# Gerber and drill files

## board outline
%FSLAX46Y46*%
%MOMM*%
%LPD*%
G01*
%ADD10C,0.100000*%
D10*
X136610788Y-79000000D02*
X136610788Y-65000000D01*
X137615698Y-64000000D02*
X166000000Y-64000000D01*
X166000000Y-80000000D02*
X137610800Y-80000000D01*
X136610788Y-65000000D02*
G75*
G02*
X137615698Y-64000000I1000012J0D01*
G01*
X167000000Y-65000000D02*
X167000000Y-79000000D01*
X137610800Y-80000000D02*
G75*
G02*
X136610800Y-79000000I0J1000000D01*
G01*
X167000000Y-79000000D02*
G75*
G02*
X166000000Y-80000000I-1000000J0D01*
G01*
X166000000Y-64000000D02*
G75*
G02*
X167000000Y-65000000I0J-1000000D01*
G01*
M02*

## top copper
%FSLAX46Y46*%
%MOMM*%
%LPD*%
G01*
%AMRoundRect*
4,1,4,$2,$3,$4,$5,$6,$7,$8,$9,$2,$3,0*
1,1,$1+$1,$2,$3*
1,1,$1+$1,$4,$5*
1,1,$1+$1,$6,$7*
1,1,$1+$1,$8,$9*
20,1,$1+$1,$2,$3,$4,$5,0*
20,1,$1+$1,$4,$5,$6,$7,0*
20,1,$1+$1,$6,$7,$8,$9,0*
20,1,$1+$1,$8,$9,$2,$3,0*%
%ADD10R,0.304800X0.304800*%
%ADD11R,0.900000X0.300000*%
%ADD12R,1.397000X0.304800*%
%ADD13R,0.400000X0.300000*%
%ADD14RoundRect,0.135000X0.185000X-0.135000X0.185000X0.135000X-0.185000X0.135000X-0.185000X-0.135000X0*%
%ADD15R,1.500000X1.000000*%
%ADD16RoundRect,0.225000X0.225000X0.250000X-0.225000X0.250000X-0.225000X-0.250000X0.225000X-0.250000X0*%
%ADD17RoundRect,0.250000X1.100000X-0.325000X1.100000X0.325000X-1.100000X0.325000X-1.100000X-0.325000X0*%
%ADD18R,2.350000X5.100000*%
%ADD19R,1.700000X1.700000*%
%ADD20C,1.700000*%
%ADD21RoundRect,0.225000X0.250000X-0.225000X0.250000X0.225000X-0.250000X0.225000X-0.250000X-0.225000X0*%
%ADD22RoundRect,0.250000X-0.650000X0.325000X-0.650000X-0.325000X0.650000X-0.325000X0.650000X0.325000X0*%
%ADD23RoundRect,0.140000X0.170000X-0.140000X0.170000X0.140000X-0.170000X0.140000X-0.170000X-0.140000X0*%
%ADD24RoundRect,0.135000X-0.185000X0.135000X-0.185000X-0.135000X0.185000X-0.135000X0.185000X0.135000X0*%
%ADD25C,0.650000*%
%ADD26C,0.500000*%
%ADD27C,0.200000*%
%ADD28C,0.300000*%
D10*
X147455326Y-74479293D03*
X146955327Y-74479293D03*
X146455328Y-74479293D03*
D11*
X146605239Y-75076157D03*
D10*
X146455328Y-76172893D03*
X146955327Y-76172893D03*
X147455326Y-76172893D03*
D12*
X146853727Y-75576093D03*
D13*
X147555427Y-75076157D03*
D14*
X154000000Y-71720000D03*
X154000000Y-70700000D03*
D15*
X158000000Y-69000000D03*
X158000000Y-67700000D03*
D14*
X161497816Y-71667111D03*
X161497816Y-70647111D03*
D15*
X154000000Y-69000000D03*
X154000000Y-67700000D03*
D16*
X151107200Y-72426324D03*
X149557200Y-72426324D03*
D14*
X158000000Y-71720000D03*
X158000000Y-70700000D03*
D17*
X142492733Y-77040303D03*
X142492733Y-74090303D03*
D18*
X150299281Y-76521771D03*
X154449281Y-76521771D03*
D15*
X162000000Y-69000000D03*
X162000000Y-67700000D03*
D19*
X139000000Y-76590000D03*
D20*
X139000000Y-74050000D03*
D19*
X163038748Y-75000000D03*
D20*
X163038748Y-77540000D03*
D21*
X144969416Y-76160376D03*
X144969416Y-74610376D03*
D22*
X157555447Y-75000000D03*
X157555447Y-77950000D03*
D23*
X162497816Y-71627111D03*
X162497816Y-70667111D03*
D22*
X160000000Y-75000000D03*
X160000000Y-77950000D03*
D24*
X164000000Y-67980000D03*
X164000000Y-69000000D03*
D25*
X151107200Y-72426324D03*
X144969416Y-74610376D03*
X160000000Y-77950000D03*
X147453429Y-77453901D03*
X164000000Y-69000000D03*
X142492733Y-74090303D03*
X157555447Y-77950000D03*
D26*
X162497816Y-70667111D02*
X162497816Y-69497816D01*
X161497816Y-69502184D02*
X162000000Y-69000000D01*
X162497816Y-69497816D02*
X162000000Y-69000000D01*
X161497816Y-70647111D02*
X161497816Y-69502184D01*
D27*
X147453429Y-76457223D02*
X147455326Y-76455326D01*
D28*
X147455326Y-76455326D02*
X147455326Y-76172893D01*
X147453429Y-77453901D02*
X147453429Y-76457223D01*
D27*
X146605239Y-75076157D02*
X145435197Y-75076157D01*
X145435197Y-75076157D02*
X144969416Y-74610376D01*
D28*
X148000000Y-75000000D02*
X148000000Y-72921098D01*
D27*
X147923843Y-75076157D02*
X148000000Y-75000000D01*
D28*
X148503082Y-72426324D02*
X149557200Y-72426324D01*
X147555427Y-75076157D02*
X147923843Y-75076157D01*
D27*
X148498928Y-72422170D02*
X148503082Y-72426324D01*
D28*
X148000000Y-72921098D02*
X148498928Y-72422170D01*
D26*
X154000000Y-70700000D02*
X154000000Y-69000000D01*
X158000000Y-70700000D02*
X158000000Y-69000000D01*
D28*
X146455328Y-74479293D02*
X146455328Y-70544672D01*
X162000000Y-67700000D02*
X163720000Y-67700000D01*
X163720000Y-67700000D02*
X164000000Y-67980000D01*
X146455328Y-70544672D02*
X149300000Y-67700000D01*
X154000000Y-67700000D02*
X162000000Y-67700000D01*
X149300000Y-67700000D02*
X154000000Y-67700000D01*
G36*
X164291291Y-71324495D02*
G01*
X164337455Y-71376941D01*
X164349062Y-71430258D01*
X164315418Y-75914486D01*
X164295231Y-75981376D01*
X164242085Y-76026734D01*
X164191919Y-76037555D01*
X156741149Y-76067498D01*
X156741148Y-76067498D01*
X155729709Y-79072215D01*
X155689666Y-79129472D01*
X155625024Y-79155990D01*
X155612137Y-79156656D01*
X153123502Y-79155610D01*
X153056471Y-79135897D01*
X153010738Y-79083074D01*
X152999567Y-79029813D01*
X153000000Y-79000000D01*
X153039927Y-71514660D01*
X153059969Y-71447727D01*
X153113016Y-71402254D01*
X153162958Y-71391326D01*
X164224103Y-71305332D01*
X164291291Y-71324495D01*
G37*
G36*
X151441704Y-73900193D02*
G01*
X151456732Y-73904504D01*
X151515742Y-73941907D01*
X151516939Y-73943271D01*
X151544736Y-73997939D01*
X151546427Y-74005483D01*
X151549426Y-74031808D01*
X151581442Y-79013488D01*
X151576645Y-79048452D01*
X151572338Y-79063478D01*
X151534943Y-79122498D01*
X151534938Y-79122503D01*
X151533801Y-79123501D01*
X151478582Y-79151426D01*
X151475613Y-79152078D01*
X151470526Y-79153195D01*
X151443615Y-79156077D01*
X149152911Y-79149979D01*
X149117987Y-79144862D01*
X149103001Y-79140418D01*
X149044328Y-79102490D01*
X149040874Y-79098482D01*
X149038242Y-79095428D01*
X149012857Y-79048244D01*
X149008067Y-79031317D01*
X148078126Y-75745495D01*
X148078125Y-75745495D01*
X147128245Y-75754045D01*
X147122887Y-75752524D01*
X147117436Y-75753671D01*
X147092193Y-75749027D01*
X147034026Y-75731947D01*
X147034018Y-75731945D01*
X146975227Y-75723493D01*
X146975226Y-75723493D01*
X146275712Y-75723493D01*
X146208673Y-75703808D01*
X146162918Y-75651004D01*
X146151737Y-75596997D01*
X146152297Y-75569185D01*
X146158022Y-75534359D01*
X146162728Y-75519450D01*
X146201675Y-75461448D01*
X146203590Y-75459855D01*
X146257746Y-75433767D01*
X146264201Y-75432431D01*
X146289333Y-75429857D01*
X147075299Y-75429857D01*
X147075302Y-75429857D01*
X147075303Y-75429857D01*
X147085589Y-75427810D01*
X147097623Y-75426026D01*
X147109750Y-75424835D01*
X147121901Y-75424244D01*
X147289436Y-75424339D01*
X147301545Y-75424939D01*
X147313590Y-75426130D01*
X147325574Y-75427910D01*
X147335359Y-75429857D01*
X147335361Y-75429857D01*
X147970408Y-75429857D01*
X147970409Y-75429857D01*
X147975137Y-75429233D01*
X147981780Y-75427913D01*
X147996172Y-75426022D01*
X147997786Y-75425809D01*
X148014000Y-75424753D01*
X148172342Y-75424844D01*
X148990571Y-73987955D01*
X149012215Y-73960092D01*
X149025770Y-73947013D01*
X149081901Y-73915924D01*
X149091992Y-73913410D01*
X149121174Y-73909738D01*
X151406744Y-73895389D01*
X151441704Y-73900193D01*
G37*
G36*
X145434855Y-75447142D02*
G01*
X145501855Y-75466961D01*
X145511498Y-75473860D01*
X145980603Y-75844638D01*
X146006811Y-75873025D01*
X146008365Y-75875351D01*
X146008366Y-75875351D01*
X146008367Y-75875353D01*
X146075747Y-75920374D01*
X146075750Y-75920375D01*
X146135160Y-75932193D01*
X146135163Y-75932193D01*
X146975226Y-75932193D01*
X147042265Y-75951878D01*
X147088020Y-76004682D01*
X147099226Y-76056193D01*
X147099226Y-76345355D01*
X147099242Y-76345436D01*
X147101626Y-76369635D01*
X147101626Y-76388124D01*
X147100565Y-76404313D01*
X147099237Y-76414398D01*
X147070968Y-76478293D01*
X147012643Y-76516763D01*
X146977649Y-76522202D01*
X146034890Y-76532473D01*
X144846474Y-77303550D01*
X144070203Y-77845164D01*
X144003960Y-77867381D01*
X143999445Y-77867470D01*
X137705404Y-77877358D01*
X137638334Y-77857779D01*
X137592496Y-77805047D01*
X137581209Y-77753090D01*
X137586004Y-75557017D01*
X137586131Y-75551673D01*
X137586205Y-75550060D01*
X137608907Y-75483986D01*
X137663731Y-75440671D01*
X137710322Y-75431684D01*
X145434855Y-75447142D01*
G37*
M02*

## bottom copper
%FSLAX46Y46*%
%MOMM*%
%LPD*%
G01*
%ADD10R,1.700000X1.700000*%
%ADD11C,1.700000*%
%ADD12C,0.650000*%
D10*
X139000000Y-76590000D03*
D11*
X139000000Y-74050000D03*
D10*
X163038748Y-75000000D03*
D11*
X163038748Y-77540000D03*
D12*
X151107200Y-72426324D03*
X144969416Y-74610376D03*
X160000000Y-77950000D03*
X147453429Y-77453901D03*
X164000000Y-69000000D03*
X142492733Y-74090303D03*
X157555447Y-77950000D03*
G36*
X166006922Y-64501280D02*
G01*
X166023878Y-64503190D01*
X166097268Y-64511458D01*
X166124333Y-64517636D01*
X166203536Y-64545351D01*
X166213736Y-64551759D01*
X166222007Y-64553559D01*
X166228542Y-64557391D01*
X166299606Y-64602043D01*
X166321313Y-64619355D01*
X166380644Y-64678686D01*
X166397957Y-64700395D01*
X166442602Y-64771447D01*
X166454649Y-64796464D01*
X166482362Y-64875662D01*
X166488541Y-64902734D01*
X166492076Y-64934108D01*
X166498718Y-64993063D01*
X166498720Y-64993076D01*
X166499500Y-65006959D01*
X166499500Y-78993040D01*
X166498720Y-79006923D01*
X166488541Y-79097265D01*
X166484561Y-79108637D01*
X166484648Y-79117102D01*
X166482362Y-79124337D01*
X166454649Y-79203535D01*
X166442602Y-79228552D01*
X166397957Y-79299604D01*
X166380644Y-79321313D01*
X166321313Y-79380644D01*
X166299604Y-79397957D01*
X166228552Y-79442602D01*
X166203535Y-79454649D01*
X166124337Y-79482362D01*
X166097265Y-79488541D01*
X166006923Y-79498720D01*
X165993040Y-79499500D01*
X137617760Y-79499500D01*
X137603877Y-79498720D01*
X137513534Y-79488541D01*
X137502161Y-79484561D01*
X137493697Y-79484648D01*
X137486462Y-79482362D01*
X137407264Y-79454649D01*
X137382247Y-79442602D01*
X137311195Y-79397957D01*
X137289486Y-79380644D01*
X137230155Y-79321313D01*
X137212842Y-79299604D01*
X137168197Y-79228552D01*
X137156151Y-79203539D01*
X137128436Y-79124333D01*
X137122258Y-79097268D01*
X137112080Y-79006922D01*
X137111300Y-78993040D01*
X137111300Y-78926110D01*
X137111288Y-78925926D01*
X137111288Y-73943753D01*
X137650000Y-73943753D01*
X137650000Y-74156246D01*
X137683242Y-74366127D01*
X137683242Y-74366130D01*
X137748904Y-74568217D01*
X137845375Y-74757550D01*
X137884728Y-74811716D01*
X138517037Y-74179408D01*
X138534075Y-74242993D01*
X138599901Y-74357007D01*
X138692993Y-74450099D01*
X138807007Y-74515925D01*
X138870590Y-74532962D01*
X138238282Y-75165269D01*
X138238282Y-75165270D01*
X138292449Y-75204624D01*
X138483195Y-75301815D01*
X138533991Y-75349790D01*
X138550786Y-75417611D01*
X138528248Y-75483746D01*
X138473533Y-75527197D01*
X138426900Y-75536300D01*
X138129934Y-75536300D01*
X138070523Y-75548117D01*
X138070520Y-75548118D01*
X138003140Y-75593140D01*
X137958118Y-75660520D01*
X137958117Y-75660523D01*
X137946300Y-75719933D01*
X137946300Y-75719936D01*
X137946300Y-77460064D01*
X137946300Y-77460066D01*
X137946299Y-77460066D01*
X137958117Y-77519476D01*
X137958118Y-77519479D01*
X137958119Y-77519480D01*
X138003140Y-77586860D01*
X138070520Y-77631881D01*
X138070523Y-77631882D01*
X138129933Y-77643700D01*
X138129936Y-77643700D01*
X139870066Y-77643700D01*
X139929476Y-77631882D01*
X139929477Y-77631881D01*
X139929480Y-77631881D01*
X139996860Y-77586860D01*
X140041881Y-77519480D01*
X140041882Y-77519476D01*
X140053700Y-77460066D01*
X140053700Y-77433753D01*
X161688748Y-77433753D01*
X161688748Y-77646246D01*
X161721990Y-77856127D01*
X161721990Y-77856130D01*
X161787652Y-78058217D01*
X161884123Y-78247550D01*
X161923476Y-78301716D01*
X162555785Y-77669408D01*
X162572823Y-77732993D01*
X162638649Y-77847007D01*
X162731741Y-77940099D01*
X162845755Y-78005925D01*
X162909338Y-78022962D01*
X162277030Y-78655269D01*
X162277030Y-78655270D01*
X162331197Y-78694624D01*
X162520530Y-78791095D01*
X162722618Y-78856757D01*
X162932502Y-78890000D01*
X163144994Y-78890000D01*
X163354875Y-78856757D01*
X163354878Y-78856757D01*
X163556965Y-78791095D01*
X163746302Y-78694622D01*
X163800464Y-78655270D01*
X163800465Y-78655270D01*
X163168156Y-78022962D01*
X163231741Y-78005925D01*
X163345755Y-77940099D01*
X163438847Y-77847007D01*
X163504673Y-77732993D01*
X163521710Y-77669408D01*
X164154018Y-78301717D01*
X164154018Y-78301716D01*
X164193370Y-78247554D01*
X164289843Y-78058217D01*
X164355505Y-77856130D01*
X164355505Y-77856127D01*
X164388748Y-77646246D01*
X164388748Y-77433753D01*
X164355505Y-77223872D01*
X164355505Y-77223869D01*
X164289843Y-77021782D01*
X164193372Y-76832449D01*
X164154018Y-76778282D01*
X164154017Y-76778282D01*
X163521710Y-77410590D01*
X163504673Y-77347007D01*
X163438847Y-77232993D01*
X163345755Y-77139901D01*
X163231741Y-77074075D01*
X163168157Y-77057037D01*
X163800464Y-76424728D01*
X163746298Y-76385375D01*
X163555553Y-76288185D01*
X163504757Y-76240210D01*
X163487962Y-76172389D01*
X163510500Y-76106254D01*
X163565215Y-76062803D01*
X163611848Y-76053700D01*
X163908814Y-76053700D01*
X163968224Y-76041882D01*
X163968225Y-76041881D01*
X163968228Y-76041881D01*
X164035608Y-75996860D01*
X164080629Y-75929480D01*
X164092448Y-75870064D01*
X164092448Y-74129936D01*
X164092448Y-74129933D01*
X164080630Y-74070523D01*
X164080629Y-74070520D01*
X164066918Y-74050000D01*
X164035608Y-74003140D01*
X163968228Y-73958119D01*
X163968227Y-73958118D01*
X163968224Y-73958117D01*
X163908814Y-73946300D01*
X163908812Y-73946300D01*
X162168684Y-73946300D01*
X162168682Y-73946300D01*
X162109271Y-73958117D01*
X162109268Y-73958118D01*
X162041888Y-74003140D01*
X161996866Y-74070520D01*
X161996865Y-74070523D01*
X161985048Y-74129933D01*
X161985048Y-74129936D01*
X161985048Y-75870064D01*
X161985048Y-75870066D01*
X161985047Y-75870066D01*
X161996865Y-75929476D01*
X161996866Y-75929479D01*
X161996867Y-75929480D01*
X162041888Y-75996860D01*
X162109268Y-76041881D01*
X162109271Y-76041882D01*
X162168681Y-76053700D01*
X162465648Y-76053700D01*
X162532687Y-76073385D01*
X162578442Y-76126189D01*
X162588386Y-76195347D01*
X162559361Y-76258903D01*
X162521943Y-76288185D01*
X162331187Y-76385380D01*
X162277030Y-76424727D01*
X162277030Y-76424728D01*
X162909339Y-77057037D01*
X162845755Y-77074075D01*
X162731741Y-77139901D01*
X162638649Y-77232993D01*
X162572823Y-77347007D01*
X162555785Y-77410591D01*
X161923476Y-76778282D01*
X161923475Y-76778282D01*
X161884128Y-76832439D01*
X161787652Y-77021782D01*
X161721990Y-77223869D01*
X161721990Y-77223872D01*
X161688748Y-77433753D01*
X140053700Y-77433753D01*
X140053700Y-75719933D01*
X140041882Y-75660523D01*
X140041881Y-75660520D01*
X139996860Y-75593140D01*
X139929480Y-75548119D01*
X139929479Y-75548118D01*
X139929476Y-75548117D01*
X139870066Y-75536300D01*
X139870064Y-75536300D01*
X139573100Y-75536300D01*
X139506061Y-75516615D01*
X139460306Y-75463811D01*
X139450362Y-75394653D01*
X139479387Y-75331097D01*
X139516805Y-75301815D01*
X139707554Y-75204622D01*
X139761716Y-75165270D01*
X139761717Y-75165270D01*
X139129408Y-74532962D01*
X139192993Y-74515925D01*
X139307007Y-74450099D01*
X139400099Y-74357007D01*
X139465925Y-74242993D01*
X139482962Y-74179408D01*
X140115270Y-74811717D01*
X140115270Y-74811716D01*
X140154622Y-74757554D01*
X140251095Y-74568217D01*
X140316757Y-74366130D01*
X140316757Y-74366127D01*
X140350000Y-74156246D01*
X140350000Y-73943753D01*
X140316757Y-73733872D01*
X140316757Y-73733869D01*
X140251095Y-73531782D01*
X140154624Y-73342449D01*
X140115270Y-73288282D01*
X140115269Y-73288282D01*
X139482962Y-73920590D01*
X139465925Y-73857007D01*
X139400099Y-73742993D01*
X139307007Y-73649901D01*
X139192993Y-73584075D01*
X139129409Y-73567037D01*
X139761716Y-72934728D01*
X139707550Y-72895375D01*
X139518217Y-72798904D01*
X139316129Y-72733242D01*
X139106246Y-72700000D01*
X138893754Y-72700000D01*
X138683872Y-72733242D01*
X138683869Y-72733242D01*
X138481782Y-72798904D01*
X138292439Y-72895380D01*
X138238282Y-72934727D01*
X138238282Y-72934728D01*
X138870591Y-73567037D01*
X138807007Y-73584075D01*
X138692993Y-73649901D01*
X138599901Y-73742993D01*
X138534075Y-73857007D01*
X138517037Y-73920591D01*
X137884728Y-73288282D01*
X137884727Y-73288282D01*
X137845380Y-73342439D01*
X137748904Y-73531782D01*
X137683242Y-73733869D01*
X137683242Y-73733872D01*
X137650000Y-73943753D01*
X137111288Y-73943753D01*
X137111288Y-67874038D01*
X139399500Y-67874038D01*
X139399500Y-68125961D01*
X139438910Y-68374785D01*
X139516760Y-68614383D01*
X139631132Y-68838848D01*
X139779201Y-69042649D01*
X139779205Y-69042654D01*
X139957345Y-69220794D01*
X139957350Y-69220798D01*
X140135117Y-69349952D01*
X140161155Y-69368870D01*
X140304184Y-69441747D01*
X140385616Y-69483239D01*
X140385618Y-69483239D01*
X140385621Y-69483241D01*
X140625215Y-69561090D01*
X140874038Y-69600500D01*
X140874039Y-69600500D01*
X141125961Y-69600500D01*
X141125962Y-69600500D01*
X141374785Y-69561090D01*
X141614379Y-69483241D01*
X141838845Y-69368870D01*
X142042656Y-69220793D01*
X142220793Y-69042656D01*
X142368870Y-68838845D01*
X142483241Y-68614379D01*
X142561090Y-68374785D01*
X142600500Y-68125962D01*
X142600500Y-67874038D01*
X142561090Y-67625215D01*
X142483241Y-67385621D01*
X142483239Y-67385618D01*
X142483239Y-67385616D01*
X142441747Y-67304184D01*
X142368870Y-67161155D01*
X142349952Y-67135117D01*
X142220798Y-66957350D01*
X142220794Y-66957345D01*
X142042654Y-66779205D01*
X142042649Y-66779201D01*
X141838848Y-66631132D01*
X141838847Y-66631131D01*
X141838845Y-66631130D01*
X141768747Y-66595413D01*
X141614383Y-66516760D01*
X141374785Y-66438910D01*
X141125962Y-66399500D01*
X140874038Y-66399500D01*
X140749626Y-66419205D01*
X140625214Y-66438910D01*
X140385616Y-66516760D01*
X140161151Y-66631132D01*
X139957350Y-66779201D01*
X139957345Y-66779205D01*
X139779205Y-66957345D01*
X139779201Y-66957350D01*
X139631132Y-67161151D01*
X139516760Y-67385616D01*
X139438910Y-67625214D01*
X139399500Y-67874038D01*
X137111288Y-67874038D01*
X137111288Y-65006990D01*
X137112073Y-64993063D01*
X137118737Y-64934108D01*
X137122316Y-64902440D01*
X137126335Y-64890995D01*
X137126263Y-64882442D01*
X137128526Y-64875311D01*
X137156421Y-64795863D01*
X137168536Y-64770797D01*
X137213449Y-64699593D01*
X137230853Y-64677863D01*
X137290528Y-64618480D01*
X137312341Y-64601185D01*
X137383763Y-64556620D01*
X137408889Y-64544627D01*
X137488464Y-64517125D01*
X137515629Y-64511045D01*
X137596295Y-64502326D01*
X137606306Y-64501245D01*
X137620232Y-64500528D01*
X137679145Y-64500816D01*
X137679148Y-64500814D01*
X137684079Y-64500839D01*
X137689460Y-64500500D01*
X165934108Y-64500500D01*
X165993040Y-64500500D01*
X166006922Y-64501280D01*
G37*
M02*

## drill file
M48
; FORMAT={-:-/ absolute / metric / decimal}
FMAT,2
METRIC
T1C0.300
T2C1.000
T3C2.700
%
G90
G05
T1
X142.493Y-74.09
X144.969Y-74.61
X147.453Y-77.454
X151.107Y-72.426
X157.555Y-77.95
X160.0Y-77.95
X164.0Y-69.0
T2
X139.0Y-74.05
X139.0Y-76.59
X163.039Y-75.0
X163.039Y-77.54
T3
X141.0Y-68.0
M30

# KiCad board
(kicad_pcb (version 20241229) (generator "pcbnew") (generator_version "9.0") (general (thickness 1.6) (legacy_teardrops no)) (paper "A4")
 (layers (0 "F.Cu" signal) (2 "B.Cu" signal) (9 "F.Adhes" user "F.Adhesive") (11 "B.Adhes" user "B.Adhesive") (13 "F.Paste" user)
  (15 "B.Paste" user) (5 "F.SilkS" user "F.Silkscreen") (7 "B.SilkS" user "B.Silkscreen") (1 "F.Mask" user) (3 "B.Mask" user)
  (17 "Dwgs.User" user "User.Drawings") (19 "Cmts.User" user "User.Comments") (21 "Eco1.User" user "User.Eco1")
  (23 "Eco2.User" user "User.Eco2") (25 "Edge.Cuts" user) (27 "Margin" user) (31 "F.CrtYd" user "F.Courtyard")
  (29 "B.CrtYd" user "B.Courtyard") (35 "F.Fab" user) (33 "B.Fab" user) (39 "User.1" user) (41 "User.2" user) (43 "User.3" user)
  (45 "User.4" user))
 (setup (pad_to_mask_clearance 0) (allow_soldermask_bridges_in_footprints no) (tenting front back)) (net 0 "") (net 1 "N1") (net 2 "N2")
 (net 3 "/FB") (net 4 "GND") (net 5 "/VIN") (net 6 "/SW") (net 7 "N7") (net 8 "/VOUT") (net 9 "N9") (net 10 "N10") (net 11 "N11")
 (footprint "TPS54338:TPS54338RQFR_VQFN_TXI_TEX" (layer "F.Cu") (at 146.955327 75.326093 -90)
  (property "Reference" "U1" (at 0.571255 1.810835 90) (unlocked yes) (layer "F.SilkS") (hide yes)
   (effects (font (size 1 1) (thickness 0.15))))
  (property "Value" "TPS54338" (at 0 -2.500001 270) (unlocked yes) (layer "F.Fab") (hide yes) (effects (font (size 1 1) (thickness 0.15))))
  (pad "1" smd rect (at -0.8468 -0.499999) (size 0.3048 0.3048) (layers "F.Cu" "F.Mask" "F.Paste") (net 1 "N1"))
  (pad "2" smd rect (at -0.8468 0) (size 0.3048 0.3048) (layers "F.Cu" "F.Mask" "F.Paste") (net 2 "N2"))
  (pad "3" smd rect (at -0.8468 0.499999) (size 0.3048 0.3048) (layers "F.Cu" "F.Mask" "F.Paste") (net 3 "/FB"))
  (pad "4" smd rect (at -0.249936 0.350088 270) (size 0.3 0.9) (layers "F.Cu" "F.Mask" "F.Paste") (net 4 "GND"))
  (pad "5" smd rect (at 0.8468 0.499999) (size 0.3048 0.3048) (layers "F.Cu" "F.Mask" "F.Paste") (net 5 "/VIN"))
  (pad "6" smd rect (at 0.8468 0) (size 0.3048 0.3048) (layers "F.Cu" "F.Mask" "F.Paste") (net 5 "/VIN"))
  (pad "7" smd rect (at 0.8468 -0.499999) (size 0.3048 0.3048) (layers "F.Cu" "F.Mask" "F.Paste") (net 4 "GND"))
  (pad "8" smd rect (at 0.25 0.1016 270) (size 0.3048 1.397) (layers "F.Cu" "F.Mask" "F.Paste") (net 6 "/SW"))
  (pad "9" smd rect (at -0.249936 -0.6001 270) (size 0.3 0.4) (layers "F.Cu" "F.Mask" "F.Paste") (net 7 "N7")))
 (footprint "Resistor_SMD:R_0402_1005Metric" (layer "F.Cu") (at 154 71.21 90)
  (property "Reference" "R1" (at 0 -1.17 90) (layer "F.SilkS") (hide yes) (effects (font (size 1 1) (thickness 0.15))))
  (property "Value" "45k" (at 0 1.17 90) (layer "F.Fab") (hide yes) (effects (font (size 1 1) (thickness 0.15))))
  (pad "1" smd roundrect (at -0.51 0 90) (size 0.54 0.64) (layers "F.Cu" "F.Mask" "F.Paste") (roundrect_rratio 0.25) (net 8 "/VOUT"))
  (pad "2" smd roundrect (at 0.51 0 90) (size 0.54 0.64) (layers "F.Cu" "F.Mask" "F.Paste") (roundrect_rratio 0.25) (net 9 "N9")))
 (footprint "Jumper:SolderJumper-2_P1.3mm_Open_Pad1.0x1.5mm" (layer "F.Cu") (at 158 68.35 90)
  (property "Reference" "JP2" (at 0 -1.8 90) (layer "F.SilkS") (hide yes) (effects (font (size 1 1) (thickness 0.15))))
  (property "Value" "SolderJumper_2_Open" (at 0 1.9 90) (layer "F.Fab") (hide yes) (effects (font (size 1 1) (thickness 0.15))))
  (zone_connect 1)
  (pad "1" smd rect (at -0.65 0 90) (size 1 1.5) (layers "F.Cu" "F.Mask") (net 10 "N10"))
  (pad "2" smd rect (at 0.65 0 90) (size 1 1.5) (layers "F.Cu" "F.Mask") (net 3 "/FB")))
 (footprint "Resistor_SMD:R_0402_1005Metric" (layer "F.Cu") (at 161.497816 71.157111 90)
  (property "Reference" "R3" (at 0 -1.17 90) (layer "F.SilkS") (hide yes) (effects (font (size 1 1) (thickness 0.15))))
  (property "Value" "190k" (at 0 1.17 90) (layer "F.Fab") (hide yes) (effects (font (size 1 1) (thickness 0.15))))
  (pad "1" smd roundrect (at -0.51 0 90) (size 0.54 0.64) (layers "F.Cu" "F.Mask" "F.Paste") (roundrect_rratio 0.25) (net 8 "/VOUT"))
  (pad "2" smd roundrect (at 0.51 0 90) (size 0.54 0.64) (layers "F.Cu" "F.Mask" "F.Paste") (roundrect_rratio 0.25) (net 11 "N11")))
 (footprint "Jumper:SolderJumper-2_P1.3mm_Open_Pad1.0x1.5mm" (layer "F.Cu") (at 154 68.35 90)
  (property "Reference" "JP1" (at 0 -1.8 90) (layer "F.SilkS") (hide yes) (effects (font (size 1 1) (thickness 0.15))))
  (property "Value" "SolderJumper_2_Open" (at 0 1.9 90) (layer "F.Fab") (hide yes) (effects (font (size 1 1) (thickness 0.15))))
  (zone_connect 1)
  (pad "1" smd rect (at -0.65 0 90) (size 1 1.5) (layers "F.Cu" "F.Mask") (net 9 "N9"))
  (pad "2" smd rect (at 0.65 0 90) (size 1 1.5) (layers "F.Cu" "F.Mask") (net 3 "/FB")))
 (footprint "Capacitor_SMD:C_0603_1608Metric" (layer "F.Cu") (at 150.3322 72.426324 180)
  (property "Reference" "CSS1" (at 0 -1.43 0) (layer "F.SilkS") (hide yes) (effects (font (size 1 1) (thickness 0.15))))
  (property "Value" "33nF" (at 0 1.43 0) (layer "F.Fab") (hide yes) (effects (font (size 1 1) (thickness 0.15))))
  (pad "1" smd roundrect (at -0.775 0 180) (size 0.9 0.95) (layers "F.Cu" "F.Mask" "F.Paste") (roundrect_rratio 0.25) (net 4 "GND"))
  (pad "2" smd roundrect (at 0.775 0 180) (size 0.9 0.95) (layers "F.Cu" "F.Mask" "F.Paste") (roundrect_rratio 0.25) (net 7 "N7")))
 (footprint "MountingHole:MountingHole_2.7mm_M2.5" (layer "F.Cu") (at 141 68)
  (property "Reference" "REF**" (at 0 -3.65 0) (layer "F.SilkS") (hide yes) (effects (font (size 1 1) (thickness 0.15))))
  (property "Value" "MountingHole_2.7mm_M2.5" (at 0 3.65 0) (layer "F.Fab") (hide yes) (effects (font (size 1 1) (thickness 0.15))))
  (pad "" np_thru_hole circle (at 0 0) (size 2.7 2.7) (drill 2.7) (layers "*.Cu" "*.Mask")))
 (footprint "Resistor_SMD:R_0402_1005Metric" (layer "F.Cu") (at 158 71.21 90)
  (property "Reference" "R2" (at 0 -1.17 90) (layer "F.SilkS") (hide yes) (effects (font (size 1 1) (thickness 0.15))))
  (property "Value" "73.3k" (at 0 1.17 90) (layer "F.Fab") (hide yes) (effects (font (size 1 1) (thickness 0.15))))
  (pad "1" smd roundrect (at -0.51 0 90) (size 0.54 0.64) (layers "F.Cu" "F.Mask" "F.Paste") (roundrect_rratio 0.25) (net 8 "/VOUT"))
  (pad "2" smd roundrect (at 0.51 0 90) (size 0.54 0.64) (layers "F.Cu" "F.Mask" "F.Paste") (roundrect_rratio 0.25) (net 10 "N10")))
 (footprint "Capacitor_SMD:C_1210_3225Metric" (layer "F.Cu") (at 142.492733 75.565303 90)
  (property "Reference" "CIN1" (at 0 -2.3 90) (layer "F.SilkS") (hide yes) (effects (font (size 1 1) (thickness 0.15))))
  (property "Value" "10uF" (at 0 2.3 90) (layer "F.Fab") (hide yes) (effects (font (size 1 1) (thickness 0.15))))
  (pad "1" smd roundrect (at -1.475 0 90) (size 1.15 2.7) (layers "F.Cu" "F.Mask" "F.Paste") (roundrect_rratio 0.217391) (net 5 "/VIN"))
  (pad "2" smd roundrect (at 1.475 0 90) (size 1.15 2.7) (layers "F.Cu" "F.Mask" "F.Paste") (roundrect_rratio 0.217391) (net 4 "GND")))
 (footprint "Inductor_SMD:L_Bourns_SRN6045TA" (layer "F.Cu") (at 152.374281 76.521771)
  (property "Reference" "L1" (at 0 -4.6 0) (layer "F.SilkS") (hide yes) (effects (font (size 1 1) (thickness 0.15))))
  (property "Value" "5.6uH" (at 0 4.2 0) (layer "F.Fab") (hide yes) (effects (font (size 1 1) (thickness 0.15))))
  (pad "1" smd rect (at -2.075 0) (size 2.35 5.1) (layers "F.Cu" "F.Mask" "F.Paste") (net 6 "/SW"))
  (pad "2" smd rect (at 2.075 0) (size 2.35 5.1) (layers "F.Cu" "F.Mask" "F.Paste") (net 8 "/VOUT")))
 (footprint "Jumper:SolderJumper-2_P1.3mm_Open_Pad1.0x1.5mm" (layer "F.Cu") (at 162 68.35 90)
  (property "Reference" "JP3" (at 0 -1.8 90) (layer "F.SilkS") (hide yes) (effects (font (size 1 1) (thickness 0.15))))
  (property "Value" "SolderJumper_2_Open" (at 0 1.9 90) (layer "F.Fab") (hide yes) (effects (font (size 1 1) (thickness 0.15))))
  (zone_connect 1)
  (pad "1" smd rect (at -0.65 0 90) (size 1 1.5) (layers "F.Cu" "F.Mask") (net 11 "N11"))
  (pad "2" smd rect (at 0.65 0 90) (size 1 1.5) (layers "F.Cu" "F.Mask") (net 3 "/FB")))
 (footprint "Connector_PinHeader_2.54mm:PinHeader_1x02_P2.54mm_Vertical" (layer "F.Cu") (at 139 76.59 180)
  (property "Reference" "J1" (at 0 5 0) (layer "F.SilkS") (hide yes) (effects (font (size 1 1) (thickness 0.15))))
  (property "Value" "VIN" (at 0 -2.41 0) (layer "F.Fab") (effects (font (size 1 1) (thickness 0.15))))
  (pad "1" thru_hole rect (at 0 0 180) (size 1.7 1.7) (drill 1) (layers "*.Cu" "*.Mask") (remove_unused_layers no) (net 5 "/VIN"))
  (pad "2" thru_hole circle (at 0 2.54 180) (size 1.7 1.7) (drill 1) (layers "*.Cu" "*.Mask") (remove_unused_layers no) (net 4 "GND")))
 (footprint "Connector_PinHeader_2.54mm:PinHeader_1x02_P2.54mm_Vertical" (layer "F.Cu") (at 163.038748 75)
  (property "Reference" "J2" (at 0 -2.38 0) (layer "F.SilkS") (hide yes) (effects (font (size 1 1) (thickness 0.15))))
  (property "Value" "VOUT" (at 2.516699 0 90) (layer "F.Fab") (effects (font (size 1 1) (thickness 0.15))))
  (pad "1" thru_hole rect (at 0 0) (size 1.7 1.7) (drill 1) (layers "*.Cu" "*.Mask") (remove_unused_layers no) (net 8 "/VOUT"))
  (pad "2" thru_hole circle (at 0 2.54) (size 1.7 1.7) (drill 1) (layers "*.Cu" "*.Mask") (remove_unused_layers no) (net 4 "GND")))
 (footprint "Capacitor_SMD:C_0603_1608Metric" (layer "F.Cu") (at 144.969416 75.385376 90)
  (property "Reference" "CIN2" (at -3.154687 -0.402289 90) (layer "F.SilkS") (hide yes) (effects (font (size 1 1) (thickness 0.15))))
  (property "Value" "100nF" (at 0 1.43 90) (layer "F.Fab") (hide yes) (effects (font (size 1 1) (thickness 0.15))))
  (pad "1" smd roundrect (at -0.775 0 90) (size 0.9 0.95) (layers "F.Cu" "F.Mask" "F.Paste") (roundrect_rratio 0.25) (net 5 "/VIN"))
  (pad "2" smd roundrect (at 0.775 0 90) (size 0.9 0.95) (layers "F.Cu" "F.Mask" "F.Paste") (roundrect_rratio 0.25) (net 4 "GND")))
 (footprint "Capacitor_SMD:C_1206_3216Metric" (layer "F.Cu") (at 157.555447 76.475 -90)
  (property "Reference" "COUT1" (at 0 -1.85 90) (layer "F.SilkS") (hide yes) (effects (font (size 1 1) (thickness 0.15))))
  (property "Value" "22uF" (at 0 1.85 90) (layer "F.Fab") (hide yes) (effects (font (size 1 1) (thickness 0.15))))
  (pad "1" smd roundrect (at -1.475 0 270) (size 1.15 1.8) (layers "F.Cu" "F.Mask" "F.Paste") (roundrect_rratio 0.217391) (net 8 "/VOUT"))
  (pad "2" smd roundrect (at 1.475 0 270) (size 1.15 1.8) (layers "F.Cu" "F.Mask" "F.Paste") (roundrect_rratio 0.217391) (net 4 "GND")))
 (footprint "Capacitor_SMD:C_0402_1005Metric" (layer "F.Cu") (at 162.497816 71.147111 90)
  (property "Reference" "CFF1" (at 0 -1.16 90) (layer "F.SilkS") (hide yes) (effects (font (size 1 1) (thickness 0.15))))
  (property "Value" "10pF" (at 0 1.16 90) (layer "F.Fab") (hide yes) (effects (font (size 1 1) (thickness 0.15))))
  (pad "1" smd roundrect (at -0.48 0 90) (size 0.56 0.62) (layers "F.Cu" "F.Mask" "F.Paste") (roundrect_rratio 0.25) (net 8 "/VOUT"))
  (pad "2" smd roundrect (at 0.48 0 90) (size 0.56 0.62) (layers "F.Cu" "F.Mask" "F.Paste") (roundrect_rratio 0.25) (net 11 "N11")))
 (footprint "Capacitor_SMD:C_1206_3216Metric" (layer "F.Cu") (at 160 76.475 -90)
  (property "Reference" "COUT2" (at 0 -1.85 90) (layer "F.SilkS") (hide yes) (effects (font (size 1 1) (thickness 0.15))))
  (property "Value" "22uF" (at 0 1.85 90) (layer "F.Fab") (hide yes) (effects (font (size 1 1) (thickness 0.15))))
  (pad "1" smd roundrect (at -1.475 0 270) (size 1.15 1.8) (layers "F.Cu" "F.Mask" "F.Paste") (roundrect_rratio 0.217391) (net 8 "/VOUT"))
  (pad "2" smd roundrect (at 1.475 0 270) (size 1.15 1.8) (layers "F.Cu" "F.Mask" "F.Paste") (roundrect_rratio 0.217391) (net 4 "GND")))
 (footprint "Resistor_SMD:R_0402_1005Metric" (layer "F.Cu") (at 164 68.49 -90)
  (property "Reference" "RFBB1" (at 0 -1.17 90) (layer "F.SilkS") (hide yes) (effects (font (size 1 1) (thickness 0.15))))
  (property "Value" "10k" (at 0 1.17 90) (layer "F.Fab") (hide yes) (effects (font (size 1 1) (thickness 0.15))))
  (pad "1" smd roundrect (at -0.51 0 270) (size 0.54 0.64) (layers "F.Cu" "F.Mask" "F.Paste") (roundrect_rratio 0.25) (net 3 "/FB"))
  (pad "2" smd roundrect (at 0.51 0 270) (size 0.54 0.64) (layers "F.Cu" "F.Mask" "F.Paste") (roundrect_rratio 0.25) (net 4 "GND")))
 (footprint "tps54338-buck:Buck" (layer "B.Cu") (at 152 70 -90)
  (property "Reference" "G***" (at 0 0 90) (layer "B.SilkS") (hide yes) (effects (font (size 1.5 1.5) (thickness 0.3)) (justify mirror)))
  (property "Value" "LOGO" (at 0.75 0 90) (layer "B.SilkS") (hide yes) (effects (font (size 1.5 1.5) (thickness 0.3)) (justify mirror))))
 (gr_line (start 136.610788 79) (end 136.610788 65) (stroke (width 0.1) (type default)) (layer "Edge.Cuts"))
 (gr_line (start 137.615698 64) (end 166 64) (stroke (width 0.1) (type default)) (layer "Edge.Cuts"))
 (gr_line (start 166 80) (end 137.6108 80) (stroke (width 0.1) (type default)) (layer "Edge.Cuts"))
 (gr_arc (start 136.610788 65) (mid 136.903681 64.292893) (end 137.615698 64) (stroke (width 0.1) (type default)) (layer "Edge.Cuts"))
 (gr_line (start 167 65) (end 167 79) (stroke (width 0.1) (type default)) (layer "Edge.Cuts"))
 (gr_arc (start 137.6108 80) (mid 136.903689 79.707103) (end 136.6108 79) (stroke (width 0.1) (type default)) (layer "Edge.Cuts"))
 (gr_arc (start 167 79) (mid 166.707107 79.707107) (end 166 80) (stroke (width 0.1) (type default)) (layer "Edge.Cuts"))
 (gr_arc (start 166 64) (mid 166.707107 64.292893) (end 167 65) (stroke (width 0.1) (type default)) (layer "Edge.Cuts"))
 (segment (start 162.497816 70.667111) (end 162.497816 69.497816) (width 0.5) (layer "F.Cu") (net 11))
 (segment (start 161.497816 69.502184) (end 162 69) (width 0.5) (layer "F.Cu") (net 11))
 (segment (start 162.497816 69.497816) (end 162 69) (width 0.5) (layer "F.Cu") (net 11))
 (segment (start 161.497816 70.647111) (end 161.497816 69.502184) (width 0.5) (layer "F.Cu") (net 11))
 (segment (start 147.453429 76.457223) (end 147.455326 76.455326) (width 0.2) (layer "F.Cu") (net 4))
 (segment (start 147.455326 76.455326) (end 147.455326 76.172893) (width 0.3) (layer "F.Cu") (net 4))
 (segment (start 147.453429 77.453901) (end 147.453429 76.457223) (width 0.3) (layer "F.Cu") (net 4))
 (segment (start 146.605239 75.076157) (end 145.435197 75.076157) (width 0.2) (layer "F.Cu") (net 4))
 (segment (start 145.435197 75.076157) (end 144.969416 74.610376) (width 0.2) (layer "F.Cu") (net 4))
 (via (at 151.1072 72.426324) (size 0.65) (drill 0.3) (layers "F.Cu" "B.Cu") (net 4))
 (via (at 144.969416 74.610376) (size 0.65) (drill 0.3) (layers "F.Cu" "B.Cu") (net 4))
 (via (at 160 77.95) (size 0.65) (drill 0.3) (layers "F.Cu" "B.Cu") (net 4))
 (via (at 147.453429 77.453901) (size 0.65) (drill 0.3) (layers "F.Cu" "B.Cu") (free yes) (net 4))
 (via (at 164 69) (size 0.65) (drill 0.3) (layers "F.Cu" "B.Cu") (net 4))
 (via (at 142.492733 74.090303) (size 0.65) (drill 0.3) (layers "F.Cu" "B.Cu") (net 4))
 (via (at 157.555447 77.95) (size 0.65) (drill 0.3) (layers "F.Cu" "B.Cu") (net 4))
 (segment (start 148 75) (end 148 72.921098) (width 0.3) (layer "F.Cu") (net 7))
 (segment (start 147.923843 75.076157) (end 148 75) (width 0.2) (layer "F.Cu") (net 7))
 (segment (start 148.503082 72.426324) (end 149.5572 72.426324) (width 0.3) (layer "F.Cu") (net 7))
 (segment (start 147.555427 75.076157) (end 147.923843 75.076157) (width 0.3) (layer "F.Cu") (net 7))
 (segment (start 148.498928 72.42217) (end 148.503082 72.426324) (width 0.2) (layer "F.Cu") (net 7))
 (segment (start 148 72.921098) (end 148.498928 72.42217) (width 0.3) (layer "F.Cu") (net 7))
 (segment (start 154 70.7) (end 154 69) (width 0.5) (layer "F.Cu") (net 9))
 (segment (start 158 70.7) (end 158 69) (width 0.5) (layer "F.Cu") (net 10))
 (segment (start 146.455328 74.479293) (end 146.455328 70.544672) (width 0.3) (layer "F.Cu") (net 3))
 (segment (start 162 67.7) (end 163.72 67.7) (width 0.3) (layer "F.Cu") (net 3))
 (segment (start 163.72 67.7) (end 164 67.98) (width 0.3) (layer "F.Cu") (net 3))
 (segment (start 146.455328 70.544672) (end 149.3 67.7) (width 0.3) (layer "F.Cu") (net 3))
 (segment (start 154 67.7) (end 162 67.7) (width 0.3) (layer "F.Cu") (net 3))
 (segment (start 149.3 67.7) (end 154 67.7) (width 0.3) (layer "F.Cu") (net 3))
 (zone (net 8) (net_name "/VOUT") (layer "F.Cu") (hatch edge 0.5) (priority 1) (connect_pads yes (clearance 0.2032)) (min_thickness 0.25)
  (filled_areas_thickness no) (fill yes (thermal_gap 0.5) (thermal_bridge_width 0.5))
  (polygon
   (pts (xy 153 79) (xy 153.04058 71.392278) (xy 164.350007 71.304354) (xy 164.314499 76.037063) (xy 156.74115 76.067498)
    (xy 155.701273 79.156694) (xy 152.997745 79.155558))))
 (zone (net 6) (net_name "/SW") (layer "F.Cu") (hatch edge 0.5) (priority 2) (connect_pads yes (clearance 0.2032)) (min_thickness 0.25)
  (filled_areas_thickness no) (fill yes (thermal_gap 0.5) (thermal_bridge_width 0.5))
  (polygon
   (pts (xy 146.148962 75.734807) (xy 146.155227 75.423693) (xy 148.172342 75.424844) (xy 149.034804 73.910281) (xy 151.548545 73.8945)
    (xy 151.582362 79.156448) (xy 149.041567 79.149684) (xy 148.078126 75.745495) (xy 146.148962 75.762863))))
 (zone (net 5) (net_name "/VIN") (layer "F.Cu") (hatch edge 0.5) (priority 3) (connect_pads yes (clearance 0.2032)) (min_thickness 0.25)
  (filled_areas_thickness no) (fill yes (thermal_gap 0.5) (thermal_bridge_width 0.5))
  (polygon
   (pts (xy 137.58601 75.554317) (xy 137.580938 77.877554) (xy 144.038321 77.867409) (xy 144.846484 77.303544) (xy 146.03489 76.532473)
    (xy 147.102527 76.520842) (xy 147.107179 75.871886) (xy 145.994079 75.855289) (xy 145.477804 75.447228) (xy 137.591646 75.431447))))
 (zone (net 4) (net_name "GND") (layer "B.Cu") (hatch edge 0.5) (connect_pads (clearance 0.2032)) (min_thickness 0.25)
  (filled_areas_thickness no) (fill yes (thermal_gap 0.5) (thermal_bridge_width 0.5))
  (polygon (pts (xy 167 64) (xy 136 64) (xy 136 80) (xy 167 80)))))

